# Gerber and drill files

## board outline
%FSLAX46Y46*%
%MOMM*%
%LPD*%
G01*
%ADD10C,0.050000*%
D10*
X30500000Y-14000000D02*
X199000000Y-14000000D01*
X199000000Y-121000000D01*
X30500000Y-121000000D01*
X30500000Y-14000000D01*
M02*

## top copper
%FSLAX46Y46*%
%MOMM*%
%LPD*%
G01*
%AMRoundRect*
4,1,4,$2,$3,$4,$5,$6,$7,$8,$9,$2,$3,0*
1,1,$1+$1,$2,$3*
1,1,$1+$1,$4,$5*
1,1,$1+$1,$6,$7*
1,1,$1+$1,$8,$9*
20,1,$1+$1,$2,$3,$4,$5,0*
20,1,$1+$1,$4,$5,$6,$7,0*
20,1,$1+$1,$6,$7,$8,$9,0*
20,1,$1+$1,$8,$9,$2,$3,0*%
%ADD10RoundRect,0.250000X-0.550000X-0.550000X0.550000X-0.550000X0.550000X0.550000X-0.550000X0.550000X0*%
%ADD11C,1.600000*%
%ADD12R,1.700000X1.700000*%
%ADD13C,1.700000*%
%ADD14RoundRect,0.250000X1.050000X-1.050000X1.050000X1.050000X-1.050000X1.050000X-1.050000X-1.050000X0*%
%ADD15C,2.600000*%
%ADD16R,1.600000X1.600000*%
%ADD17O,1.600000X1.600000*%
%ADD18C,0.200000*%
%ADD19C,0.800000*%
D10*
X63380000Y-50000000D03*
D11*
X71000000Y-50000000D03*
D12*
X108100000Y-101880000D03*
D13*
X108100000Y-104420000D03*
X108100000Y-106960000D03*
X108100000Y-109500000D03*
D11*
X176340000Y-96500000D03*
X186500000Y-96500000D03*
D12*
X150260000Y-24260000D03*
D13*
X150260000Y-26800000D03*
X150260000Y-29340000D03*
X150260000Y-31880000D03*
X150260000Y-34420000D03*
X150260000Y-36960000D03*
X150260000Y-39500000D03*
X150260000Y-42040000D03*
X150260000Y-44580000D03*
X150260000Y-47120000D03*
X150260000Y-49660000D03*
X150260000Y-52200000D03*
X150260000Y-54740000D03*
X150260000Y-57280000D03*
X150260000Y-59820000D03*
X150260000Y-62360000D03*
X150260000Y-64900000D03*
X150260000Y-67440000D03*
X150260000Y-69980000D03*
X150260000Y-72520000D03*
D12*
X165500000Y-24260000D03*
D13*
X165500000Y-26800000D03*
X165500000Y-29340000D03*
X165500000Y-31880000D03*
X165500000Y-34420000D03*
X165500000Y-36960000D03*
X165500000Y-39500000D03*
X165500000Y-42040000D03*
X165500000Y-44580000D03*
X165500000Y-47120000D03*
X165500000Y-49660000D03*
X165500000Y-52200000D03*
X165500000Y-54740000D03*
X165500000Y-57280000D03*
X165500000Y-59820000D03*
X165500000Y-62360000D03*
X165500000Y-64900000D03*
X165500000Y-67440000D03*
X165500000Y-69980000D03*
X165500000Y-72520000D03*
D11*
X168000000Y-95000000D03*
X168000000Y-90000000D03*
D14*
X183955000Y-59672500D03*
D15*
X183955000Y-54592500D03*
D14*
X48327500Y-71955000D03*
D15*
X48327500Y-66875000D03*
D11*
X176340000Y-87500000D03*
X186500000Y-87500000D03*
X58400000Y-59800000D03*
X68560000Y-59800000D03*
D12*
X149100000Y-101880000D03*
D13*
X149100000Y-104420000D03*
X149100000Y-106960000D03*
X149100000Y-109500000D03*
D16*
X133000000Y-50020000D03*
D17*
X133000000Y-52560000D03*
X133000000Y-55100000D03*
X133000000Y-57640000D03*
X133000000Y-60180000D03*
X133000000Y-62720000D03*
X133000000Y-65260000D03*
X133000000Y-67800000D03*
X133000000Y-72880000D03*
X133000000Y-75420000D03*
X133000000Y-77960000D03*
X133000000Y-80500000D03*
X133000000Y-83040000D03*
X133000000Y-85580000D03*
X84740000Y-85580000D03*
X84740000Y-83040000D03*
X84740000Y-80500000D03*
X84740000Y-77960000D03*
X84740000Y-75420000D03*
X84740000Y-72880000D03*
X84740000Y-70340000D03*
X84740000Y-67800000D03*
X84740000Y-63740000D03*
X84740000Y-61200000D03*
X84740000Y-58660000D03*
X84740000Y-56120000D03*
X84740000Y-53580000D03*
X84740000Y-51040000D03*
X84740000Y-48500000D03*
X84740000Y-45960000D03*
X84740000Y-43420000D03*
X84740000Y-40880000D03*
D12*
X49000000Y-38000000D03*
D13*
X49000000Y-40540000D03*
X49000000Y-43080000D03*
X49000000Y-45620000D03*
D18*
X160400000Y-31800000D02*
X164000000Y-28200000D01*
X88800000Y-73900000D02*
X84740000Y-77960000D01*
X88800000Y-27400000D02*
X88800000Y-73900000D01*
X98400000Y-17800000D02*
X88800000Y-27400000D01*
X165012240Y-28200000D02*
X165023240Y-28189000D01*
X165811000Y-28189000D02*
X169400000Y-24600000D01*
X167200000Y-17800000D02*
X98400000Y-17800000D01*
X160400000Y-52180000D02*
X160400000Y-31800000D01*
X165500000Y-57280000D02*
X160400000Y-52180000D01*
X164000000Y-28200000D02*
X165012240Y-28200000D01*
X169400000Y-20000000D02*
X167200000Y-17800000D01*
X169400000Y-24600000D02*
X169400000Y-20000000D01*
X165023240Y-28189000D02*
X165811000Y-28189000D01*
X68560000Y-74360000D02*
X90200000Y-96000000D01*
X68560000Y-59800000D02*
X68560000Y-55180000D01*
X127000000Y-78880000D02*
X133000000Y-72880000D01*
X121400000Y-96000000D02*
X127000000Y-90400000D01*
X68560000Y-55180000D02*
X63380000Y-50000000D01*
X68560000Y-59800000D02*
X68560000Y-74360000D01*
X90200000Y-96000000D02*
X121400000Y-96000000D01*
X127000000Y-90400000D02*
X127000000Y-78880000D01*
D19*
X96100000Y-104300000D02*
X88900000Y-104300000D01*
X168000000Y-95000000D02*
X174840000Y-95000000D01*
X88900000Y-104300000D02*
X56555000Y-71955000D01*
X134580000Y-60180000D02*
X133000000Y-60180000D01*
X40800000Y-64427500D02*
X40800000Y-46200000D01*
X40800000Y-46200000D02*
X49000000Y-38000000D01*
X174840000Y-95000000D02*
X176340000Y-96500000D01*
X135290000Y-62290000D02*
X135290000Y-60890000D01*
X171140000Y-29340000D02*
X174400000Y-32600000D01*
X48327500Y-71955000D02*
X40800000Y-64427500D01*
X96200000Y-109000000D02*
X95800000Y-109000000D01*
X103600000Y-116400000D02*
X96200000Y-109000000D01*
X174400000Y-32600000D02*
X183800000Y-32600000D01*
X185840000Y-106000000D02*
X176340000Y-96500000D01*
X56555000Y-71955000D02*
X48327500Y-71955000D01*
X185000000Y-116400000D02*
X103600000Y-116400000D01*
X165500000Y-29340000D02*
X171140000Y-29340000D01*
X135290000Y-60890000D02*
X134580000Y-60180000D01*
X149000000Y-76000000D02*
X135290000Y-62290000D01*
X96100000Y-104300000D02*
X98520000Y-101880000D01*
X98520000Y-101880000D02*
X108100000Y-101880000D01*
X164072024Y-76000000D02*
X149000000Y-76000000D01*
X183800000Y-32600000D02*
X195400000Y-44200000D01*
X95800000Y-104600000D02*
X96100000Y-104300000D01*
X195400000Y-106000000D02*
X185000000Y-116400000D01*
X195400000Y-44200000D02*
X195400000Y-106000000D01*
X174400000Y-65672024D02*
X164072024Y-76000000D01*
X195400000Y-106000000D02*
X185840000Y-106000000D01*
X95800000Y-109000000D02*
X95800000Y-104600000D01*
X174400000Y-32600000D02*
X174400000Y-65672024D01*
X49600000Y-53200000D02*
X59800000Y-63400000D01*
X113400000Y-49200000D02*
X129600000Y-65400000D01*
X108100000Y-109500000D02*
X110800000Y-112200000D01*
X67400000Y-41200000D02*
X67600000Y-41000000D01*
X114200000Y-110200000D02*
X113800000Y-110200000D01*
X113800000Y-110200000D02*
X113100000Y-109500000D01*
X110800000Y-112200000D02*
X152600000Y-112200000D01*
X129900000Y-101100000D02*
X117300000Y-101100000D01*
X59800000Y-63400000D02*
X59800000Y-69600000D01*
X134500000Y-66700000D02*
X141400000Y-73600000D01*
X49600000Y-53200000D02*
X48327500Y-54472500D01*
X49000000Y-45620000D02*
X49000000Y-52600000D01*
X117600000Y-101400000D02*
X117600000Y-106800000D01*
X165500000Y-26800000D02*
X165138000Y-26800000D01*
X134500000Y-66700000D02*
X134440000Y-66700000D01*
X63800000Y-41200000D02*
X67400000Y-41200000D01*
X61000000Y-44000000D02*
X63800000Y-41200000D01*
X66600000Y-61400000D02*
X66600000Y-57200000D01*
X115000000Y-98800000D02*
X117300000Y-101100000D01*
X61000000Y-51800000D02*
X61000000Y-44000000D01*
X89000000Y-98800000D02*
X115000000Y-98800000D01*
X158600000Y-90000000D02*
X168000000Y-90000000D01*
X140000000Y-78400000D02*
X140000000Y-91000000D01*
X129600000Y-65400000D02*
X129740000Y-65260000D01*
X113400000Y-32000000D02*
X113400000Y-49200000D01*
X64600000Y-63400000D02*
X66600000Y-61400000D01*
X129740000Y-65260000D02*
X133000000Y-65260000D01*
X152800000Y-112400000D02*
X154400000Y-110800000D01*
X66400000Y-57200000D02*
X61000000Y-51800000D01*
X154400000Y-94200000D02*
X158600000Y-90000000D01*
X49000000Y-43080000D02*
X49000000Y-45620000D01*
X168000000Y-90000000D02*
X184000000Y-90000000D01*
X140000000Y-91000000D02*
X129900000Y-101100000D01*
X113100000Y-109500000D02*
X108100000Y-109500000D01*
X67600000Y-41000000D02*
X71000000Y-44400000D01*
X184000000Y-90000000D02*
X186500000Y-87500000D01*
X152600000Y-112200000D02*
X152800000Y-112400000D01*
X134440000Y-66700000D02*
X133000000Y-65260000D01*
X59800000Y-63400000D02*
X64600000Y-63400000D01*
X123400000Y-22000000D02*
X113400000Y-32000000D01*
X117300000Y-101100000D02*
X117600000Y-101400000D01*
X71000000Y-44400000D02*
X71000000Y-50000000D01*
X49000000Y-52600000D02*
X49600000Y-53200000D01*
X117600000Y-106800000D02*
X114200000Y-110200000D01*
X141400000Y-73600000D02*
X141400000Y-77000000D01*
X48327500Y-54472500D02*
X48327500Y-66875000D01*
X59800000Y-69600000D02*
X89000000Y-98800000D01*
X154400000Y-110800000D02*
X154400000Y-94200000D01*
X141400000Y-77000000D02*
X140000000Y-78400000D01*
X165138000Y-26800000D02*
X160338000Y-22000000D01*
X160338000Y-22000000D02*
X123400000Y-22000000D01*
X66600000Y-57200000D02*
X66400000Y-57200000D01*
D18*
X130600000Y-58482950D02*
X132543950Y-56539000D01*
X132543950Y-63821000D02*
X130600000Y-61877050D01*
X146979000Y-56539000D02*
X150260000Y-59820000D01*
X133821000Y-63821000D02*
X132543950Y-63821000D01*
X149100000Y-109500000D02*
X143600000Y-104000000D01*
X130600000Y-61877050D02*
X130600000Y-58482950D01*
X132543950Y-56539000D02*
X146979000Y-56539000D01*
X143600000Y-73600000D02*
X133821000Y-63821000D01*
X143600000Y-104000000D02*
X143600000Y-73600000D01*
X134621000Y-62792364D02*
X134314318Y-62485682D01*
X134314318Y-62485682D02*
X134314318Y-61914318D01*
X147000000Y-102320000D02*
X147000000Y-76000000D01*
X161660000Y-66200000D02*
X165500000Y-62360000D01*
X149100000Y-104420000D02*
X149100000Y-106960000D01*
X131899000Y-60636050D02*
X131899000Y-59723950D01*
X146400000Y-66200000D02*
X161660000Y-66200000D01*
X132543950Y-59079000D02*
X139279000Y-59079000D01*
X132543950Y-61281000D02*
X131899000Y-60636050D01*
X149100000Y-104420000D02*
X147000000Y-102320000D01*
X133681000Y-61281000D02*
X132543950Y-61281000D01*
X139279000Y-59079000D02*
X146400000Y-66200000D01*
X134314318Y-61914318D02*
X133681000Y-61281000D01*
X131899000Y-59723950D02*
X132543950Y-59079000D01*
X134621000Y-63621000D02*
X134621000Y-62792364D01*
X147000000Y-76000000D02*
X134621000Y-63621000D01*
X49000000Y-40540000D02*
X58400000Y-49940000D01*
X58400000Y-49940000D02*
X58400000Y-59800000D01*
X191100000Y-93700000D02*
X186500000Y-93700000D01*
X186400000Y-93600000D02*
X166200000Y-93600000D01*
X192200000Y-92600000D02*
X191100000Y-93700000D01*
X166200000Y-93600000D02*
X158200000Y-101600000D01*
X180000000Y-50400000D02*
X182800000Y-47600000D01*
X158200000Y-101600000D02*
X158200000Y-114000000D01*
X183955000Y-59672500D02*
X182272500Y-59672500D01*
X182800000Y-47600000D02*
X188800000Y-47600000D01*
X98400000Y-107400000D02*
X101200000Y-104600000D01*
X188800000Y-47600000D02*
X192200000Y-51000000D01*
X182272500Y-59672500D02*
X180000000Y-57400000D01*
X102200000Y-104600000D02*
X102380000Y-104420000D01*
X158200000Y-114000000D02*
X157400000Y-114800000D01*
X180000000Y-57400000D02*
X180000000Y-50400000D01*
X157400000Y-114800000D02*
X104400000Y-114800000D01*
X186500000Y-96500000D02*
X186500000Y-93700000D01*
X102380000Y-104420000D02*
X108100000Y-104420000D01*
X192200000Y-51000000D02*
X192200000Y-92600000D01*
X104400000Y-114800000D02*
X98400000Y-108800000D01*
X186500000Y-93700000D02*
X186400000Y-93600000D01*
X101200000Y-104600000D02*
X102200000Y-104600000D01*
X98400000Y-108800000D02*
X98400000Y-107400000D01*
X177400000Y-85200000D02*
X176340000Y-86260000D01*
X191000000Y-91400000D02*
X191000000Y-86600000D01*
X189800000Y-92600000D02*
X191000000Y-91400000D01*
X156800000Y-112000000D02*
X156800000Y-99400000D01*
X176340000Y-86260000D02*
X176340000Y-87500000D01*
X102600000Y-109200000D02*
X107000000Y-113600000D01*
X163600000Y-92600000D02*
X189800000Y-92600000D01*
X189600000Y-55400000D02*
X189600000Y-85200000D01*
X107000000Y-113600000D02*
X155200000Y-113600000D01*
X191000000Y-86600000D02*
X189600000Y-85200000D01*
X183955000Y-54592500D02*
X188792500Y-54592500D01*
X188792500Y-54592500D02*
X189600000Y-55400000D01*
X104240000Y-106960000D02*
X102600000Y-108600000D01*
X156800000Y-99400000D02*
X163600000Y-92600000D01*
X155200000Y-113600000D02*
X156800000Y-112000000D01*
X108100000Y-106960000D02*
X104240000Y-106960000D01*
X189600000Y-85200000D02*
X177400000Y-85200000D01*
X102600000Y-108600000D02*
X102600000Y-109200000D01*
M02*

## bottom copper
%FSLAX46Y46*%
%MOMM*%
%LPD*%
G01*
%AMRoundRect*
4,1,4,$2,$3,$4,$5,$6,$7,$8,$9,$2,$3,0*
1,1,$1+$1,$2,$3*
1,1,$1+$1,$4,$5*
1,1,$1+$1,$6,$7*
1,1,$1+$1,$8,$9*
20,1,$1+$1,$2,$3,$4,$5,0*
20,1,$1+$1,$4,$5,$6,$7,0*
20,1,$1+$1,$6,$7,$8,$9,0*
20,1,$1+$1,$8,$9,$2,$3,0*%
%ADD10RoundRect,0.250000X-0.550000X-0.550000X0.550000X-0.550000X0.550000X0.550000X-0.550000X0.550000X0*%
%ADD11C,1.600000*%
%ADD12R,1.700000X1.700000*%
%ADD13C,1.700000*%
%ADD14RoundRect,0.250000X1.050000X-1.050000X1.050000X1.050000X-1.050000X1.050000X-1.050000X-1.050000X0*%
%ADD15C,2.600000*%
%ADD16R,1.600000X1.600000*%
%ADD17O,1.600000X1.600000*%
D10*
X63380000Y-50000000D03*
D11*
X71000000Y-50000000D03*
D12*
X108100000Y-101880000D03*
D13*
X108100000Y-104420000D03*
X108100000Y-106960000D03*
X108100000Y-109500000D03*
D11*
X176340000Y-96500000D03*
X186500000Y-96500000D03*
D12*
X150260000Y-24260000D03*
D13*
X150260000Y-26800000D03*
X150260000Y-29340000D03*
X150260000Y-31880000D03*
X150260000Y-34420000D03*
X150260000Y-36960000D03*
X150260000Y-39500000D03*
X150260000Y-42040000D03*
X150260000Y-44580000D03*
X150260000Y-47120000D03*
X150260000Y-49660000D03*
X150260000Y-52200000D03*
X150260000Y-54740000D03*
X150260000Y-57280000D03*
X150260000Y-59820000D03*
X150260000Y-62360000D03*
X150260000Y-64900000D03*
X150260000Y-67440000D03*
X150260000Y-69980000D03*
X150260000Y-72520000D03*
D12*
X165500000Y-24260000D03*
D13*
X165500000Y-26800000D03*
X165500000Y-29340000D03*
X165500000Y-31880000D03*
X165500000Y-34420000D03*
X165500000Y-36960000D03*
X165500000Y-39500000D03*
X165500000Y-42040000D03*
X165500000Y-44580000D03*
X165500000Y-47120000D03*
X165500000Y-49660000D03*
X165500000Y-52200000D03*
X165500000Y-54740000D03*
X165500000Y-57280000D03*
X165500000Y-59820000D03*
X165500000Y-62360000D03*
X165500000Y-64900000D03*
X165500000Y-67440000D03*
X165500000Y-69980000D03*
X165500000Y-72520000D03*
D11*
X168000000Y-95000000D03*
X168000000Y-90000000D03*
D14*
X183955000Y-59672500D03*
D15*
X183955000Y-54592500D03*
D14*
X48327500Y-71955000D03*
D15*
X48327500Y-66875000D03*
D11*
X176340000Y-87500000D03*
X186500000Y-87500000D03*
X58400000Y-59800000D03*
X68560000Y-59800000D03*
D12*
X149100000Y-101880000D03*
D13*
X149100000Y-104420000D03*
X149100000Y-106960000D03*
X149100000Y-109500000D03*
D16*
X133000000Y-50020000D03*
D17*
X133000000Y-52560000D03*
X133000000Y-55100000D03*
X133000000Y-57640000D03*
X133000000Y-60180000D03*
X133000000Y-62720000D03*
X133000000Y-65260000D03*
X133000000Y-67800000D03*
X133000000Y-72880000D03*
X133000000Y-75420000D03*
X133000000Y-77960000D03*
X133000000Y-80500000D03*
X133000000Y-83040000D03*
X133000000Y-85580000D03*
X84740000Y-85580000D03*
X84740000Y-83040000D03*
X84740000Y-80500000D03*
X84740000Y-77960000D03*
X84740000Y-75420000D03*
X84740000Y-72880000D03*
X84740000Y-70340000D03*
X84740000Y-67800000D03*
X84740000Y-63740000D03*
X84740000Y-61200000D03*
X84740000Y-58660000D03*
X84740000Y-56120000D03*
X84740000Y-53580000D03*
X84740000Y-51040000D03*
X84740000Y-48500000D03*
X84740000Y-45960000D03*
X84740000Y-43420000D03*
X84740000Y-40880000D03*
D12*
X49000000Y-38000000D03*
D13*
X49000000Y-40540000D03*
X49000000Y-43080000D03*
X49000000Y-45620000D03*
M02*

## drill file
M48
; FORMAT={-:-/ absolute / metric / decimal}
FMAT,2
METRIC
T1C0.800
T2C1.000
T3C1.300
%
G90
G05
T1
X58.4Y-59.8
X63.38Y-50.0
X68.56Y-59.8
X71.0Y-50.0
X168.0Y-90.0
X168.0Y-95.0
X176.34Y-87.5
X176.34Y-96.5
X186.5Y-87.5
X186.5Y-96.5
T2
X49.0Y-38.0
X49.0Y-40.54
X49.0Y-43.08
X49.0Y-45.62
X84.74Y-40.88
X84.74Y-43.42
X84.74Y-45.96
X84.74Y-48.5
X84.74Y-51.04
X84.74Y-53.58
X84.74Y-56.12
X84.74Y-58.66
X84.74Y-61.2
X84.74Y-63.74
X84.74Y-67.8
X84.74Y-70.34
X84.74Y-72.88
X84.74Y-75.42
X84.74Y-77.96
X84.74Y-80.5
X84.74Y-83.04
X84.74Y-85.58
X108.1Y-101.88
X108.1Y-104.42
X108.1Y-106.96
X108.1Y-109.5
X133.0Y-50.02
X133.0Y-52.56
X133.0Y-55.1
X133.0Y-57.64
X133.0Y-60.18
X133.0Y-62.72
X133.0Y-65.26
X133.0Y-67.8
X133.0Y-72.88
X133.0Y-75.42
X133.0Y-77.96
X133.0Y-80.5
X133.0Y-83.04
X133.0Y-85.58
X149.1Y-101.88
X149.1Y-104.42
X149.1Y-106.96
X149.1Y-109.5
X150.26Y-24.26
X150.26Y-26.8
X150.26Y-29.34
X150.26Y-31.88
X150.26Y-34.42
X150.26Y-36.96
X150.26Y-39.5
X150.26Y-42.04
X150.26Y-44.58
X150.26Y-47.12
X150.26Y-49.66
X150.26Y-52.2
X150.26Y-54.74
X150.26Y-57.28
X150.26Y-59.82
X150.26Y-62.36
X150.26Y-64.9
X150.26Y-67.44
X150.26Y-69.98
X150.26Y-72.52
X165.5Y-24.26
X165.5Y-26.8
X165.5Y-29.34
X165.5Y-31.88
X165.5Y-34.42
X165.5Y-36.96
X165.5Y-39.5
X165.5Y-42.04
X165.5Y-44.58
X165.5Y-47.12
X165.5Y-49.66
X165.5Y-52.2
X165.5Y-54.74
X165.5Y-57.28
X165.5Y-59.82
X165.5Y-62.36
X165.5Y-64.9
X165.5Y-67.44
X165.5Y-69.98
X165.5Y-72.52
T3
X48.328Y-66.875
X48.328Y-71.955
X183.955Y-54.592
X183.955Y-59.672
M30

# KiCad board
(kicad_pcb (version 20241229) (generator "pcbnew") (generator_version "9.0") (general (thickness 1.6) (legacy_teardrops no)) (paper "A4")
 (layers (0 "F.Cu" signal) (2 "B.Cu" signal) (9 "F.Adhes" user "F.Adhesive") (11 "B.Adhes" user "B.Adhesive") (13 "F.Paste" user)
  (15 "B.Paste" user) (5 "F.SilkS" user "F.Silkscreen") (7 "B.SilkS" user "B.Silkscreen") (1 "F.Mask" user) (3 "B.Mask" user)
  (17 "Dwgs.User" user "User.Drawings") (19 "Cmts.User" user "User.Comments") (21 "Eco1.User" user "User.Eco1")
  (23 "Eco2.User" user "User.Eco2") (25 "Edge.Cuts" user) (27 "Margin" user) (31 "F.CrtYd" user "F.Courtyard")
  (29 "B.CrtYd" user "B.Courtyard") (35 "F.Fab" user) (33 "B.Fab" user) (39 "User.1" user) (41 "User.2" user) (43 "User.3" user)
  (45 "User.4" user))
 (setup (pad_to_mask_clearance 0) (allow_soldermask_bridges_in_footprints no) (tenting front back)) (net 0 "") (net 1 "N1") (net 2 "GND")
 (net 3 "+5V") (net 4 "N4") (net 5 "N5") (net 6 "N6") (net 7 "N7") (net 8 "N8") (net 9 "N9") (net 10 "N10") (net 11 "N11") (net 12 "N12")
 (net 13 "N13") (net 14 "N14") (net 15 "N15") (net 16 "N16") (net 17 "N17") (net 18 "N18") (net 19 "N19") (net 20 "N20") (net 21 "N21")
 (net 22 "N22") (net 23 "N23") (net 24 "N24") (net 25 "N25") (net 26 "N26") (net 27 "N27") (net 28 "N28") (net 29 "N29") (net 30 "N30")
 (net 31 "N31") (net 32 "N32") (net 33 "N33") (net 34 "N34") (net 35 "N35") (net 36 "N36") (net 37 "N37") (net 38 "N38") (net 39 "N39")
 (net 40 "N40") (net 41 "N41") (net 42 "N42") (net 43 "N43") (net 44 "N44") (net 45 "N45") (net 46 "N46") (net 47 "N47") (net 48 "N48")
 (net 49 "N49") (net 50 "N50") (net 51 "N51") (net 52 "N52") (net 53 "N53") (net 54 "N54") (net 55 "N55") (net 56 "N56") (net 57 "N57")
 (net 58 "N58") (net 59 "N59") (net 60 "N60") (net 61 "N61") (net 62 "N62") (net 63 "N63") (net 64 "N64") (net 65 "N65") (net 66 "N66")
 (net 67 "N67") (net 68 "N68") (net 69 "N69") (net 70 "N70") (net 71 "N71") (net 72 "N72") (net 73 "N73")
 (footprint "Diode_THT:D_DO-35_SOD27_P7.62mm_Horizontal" (layer "F.Cu") (at 63.38 50)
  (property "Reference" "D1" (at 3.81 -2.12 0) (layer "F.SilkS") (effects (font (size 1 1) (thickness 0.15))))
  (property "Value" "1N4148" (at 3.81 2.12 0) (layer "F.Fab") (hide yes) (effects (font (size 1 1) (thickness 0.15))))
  (pad "1" thru_hole roundrect (at 0 0) (size 1.6 1.6) (drill 0.8) (layers "*.Cu" "*.Mask") (remove_unused_layers no)
   (roundrect_rratio 0.15625) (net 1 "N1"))
  (pad "2" thru_hole circle (at 7.62 0) (size 1.6 1.6) (drill 0.8) (layers "*.Cu" "*.Mask") (remove_unused_layers no) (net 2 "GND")))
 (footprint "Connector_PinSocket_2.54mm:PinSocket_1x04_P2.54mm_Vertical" (layer "F.Cu") (at 108.1 101.88)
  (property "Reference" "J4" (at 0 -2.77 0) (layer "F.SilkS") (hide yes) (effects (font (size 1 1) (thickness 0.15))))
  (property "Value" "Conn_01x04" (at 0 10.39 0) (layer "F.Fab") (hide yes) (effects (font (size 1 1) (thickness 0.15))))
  (pad "1" thru_hole rect (at 0 0) (size 1.7 1.7) (drill 1) (layers "*.Cu" "*.Mask") (remove_unused_layers no) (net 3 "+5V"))
  (pad "2" thru_hole circle (at 0 2.54) (size 1.7 1.7) (drill 1) (layers "*.Cu" "*.Mask") (remove_unused_layers no) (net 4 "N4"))
  (pad "3" thru_hole circle (at 0 5.08) (size 1.7 1.7) (drill 1) (layers "*.Cu" "*.Mask") (remove_unused_layers no) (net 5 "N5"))
  (pad "4" thru_hole circle (at 0 7.62) (size 1.7 1.7) (drill 1) (layers "*.Cu" "*.Mask") (remove_unused_layers no) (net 2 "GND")))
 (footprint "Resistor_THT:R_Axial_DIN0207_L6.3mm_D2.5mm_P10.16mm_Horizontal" (layer "F.Cu") (at 176.34 96.5)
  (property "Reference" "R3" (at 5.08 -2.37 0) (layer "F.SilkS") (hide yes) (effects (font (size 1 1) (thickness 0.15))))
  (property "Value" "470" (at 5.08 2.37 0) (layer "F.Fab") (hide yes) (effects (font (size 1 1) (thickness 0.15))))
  (pad "1" thru_hole circle (at 0 0) (size 1.6 1.6) (drill 0.8) (layers "*.Cu" "*.Mask") (remove_unused_layers no) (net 3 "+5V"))
  (pad "2" thru_hole circle (at 10.16 0) (size 1.6 1.6) (drill 0.8) (layers "*.Cu" "*.Mask") (remove_unused_layers no) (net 4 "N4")))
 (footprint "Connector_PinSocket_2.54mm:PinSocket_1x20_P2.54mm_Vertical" (layer "F.Cu") (at 150.26 24.26)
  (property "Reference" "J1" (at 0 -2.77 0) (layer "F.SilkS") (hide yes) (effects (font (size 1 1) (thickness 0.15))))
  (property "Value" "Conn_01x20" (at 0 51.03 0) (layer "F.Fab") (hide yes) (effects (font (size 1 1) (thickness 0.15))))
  (pad "1" thru_hole rect (at 0 0) (size 1.7 1.7) (drill 1) (layers "*.Cu" "*.Mask") (remove_unused_layers no) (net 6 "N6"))
  (pad "2" thru_hole circle (at 0 2.54) (size 1.7 1.7) (drill 1) (layers "*.Cu" "*.Mask") (remove_unused_layers no) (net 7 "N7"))
  (pad "3" thru_hole circle (at 0 5.08) (size 1.7 1.7) (drill 1) (layers "*.Cu" "*.Mask") (remove_unused_layers no) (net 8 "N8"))
  (pad "4" thru_hole circle (at 0 7.62) (size 1.7 1.7) (drill 1) (layers "*.Cu" "*.Mask") (remove_unused_layers no) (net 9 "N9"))
  (pad "5" thru_hole circle (at 0 10.16) (size 1.7 1.7) (drill 1) (layers "*.Cu" "*.Mask") (remove_unused_layers no) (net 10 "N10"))
  (pad "6" thru_hole circle (at 0 12.7) (size 1.7 1.7) (drill 1) (layers "*.Cu" "*.Mask") (remove_unused_layers no) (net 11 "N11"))
  (pad "7" thru_hole circle (at 0 15.24) (size 1.7 1.7) (drill 1) (layers "*.Cu" "*.Mask") (remove_unused_layers no) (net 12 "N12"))
  (pad "8" thru_hole circle (at 0 17.78) (size 1.7 1.7) (drill 1) (layers "*.Cu" "*.Mask") (remove_unused_layers no) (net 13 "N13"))
  (pad "9" thru_hole circle (at 0 20.32) (size 1.7 1.7) (drill 1) (layers "*.Cu" "*.Mask") (remove_unused_layers no) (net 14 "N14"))
  (pad "10" thru_hole circle (at 0 22.86) (size 1.7 1.7) (drill 1) (layers "*.Cu" "*.Mask") (remove_unused_layers no) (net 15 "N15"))
  (pad "11" thru_hole circle (at 0 25.4) (size 1.7 1.7) (drill 1) (layers "*.Cu" "*.Mask") (remove_unused_layers no) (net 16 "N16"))
  (pad "12" thru_hole circle (at 0 27.94) (size 1.7 1.7) (drill 1) (layers "*.Cu" "*.Mask") (remove_unused_layers no) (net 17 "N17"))
  (pad "13" thru_hole circle (at 0 30.48) (size 1.7 1.7) (drill 1) (layers "*.Cu" "*.Mask") (remove_unused_layers no) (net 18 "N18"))
  (pad "14" thru_hole circle (at 0 33.02) (size 1.7 1.7) (drill 1) (layers "*.Cu" "*.Mask") (remove_unused_layers no) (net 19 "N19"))
  (pad "15" thru_hole circle (at 0 35.56) (size 1.7 1.7) (drill 1) (layers "*.Cu" "*.Mask") (remove_unused_layers no) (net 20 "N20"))
  (pad "16" thru_hole circle (at 0 38.1) (size 1.7 1.7) (drill 1) (layers "*.Cu" "*.Mask") (remove_unused_layers no) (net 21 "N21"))
  (pad "17" thru_hole circle (at 0 40.64) (size 1.7 1.7) (drill 1) (layers "*.Cu" "*.Mask") (remove_unused_layers no) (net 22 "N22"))
  (pad "18" thru_hole circle (at 0 43.18) (size 1.7 1.7) (drill 1) (layers "*.Cu" "*.Mask") (remove_unused_layers no) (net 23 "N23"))
  (pad "19" thru_hole circle (at 0 45.72) (size 1.7 1.7) (drill 1) (layers "*.Cu" "*.Mask") (remove_unused_layers no) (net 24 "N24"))
  (pad "20" thru_hole circle (at 0 48.26) (size 1.7 1.7) (drill 1) (layers "*.Cu" "*.Mask") (remove_unused_layers no) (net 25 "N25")))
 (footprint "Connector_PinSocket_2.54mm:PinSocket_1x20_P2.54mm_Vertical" (layer "F.Cu") (at 165.5 24.26)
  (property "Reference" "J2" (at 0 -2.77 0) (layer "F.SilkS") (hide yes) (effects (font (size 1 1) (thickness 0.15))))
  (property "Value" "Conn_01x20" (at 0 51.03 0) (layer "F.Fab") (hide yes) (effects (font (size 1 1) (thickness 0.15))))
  (pad "1" thru_hole rect (at 0 0) (size 1.7 1.7) (drill 1) (layers "*.Cu" "*.Mask") (remove_unused_layers no) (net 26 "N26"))
  (pad "2" thru_hole circle (at 0 2.54) (size 1.7 1.7) (drill 1) (layers "*.Cu" "*.Mask") (remove_unused_layers no) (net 2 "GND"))
  (pad "3" thru_hole circle (at 0 5.08) (size 1.7 1.7) (drill 1) (layers "*.Cu" "*.Mask") (remove_unused_layers no) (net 3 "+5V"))
  (pad "4" thru_hole circle (at 0 7.62) (size 1.7 1.7) (drill 1) (layers "*.Cu" "*.Mask") (remove_unused_layers no) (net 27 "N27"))
  (pad "5" thru_hole circle (at 0 10.16) (size 1.7 1.7) (drill 1) (layers "*.Cu" "*.Mask") (remove_unused_layers no) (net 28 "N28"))
  (pad "6" thru_hole circle (at 0 12.7) (size 1.7 1.7) (drill 1) (layers "*.Cu" "*.Mask") (remove_unused_layers no) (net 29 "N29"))
  (pad "7" thru_hole circle (at 0 15.24) (size 1.7 1.7) (drill 1) (layers "*.Cu" "*.Mask") (remove_unused_layers no) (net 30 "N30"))
  (pad "8" thru_hole circle (at 0 17.78) (size 1.7 1.7) (drill 1) (layers "*.Cu" "*.Mask") (remove_unused_layers no) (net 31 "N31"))
  (pad "9" thru_hole circle (at 0 20.32) (size 1.7 1.7) (drill 1) (layers "*.Cu" "*.Mask") (remove_unused_layers no) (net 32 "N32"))
  (pad "10" thru_hole circle (at 0 22.86) (size 1.7 1.7) (drill 1) (layers "*.Cu" "*.Mask") (remove_unused_layers no) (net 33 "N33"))
  (pad "11" thru_hole circle (at 0 25.4) (size 1.7 1.7) (drill 1) (layers "*.Cu" "*.Mask") (remove_unused_layers no) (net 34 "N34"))
  (pad "12" thru_hole circle (at 0 27.94) (size 1.7 1.7) (drill 1) (layers "*.Cu" "*.Mask") (remove_unused_layers no) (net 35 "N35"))
  (pad "13" thru_hole circle (at 0 30.48) (size 1.7 1.7) (drill 1) (layers "*.Cu" "*.Mask") (remove_unused_layers no) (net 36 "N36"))
  (pad "14" thru_hole circle (at 0 33.02) (size 1.7 1.7) (drill 1) (layers "*.Cu" "*.Mask") (remove_unused_layers no) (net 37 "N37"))
  (pad "15" thru_hole circle (at 0 35.56) (size 1.7 1.7) (drill 1) (layers "*.Cu" "*.Mask") (remove_unused_layers no) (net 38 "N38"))
  (pad "16" thru_hole circle (at 0 38.1) (size 1.7 1.7) (drill 1) (layers "*.Cu" "*.Mask") (remove_unused_layers no) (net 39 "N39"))
  (pad "17" thru_hole circle (at 0 40.64) (size 1.7 1.7) (drill 1) (layers "*.Cu" "*.Mask") (remove_unused_layers no) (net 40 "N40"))
  (pad "18" thru_hole circle (at 0 43.18) (size 1.7 1.7) (drill 1) (layers "*.Cu" "*.Mask") (remove_unused_layers no) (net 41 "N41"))
  (pad "19" thru_hole circle (at 0 45.72) (size 1.7 1.7) (drill 1) (layers "*.Cu" "*.Mask") (remove_unused_layers no) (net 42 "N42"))
  (pad "20" thru_hole circle (at 0 48.26) (size 1.7 1.7) (drill 1) (layers "*.Cu" "*.Mask") (remove_unused_layers no) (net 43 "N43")))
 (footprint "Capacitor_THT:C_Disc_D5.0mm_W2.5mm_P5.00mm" (layer "F.Cu") (at 168 95 90)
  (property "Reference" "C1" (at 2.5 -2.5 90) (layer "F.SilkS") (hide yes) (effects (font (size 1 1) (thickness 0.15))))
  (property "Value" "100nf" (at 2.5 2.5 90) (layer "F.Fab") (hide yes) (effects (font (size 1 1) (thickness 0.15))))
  (pad "1" thru_hole circle (at 0 0 90) (size 1.6 1.6) (drill 0.8) (layers "*.Cu" "*.Mask") (remove_unused_layers no) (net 3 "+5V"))
  (pad "2" thru_hole circle (at 5 0 90) (size 1.6 1.6) (drill 0.8) (layers "*.Cu" "*.Mask") (remove_unused_layers no) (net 2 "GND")))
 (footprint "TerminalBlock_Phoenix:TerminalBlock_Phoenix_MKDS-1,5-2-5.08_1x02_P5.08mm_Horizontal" (layer "F.Cu") (at 183.955 59.6725 90)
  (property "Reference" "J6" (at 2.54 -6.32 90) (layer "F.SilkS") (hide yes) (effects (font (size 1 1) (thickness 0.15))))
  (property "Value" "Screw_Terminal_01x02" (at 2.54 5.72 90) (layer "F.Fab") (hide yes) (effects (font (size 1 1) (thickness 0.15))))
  (pad "1" thru_hole roundrect (at 0 0 90) (size 2.6 2.6) (drill 1.3) (layers "*.Cu" "*.Mask") (remove_unused_layers no)
   (roundrect_rratio 0.096154) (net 4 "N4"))
  (pad "2" thru_hole circle (at 5.08 0 90) (size 2.6 2.6) (drill 1.3) (layers "*.Cu" "*.Mask") (remove_unused_layers no) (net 5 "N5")))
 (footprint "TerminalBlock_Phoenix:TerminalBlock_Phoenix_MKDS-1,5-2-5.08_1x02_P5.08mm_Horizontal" (layer "F.Cu") (at 48.3275 71.955 90)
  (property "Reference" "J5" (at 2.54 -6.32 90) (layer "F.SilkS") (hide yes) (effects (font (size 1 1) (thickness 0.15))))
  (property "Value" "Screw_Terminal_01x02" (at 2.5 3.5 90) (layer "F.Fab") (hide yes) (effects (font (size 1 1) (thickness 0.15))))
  (pad "1" thru_hole roundrect (at 0 0 90) (size 2.6 2.6) (drill 1.3) (layers "*.Cu" "*.Mask") (remove_unused_layers no)
   (roundrect_rratio 0.096154) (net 3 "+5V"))
  (pad "2" thru_hole circle (at 5.08 0 90) (size 2.6 2.6) (drill 1.3) (layers "*.Cu" "*.Mask") (remove_unused_layers no) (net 2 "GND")))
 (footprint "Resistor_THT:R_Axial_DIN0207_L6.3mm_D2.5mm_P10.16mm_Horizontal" (layer "F.Cu") (at 176.34 87.5)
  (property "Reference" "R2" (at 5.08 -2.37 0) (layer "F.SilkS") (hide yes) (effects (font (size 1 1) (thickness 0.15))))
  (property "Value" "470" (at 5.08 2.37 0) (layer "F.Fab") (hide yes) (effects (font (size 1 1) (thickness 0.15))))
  (pad "1" thru_hole circle (at 0 0) (size 1.6 1.6) (drill 0.8) (layers "*.Cu" "*.Mask") (remove_unused_layers no) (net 5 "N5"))
  (pad "2" thru_hole circle (at 10.16 0) (size 1.6 1.6) (drill 0.8) (layers "*.Cu" "*.Mask") (remove_unused_layers no) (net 2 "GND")))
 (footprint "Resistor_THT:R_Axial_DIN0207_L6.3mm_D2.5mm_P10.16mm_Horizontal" (layer "F.Cu") (at 58.4 59.8)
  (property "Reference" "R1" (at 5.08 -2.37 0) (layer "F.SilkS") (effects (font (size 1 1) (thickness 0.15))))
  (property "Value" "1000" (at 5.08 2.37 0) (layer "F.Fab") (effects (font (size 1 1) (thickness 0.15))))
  (pad "1" thru_hole circle (at 0 0) (size 1.6 1.6) (drill 0.8) (layers "*.Cu" "*.Mask") (remove_unused_layers no) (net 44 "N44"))
  (pad "2" thru_hole circle (at 10.16 0) (size 1.6 1.6) (drill 0.8) (layers "*.Cu" "*.Mask") (remove_unused_layers no) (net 1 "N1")))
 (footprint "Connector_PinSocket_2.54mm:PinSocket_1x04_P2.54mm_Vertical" (layer "F.Cu") (at 149.1 101.88)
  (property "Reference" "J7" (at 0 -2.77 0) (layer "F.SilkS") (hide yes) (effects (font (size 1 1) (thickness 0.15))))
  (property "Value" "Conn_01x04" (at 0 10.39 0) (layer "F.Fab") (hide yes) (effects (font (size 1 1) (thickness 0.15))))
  (pad "1" thru_hole rect (at 0 0) (size 1.7 1.7) (drill 1) (layers "*.Cu" "*.Mask") (remove_unused_layers no) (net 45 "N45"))
  (pad "2" thru_hole circle (at 0 2.54) (size 1.7 1.7) (drill 1) (layers "*.Cu" "*.Mask") (remove_unused_layers no) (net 39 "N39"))
  (pad "3" thru_hole circle (at 0 5.08) (size 1.7 1.7) (drill 1) (layers "*.Cu" "*.Mask") (remove_unused_layers no) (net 39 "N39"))
  (pad "4" thru_hole circle (at 0 7.62) (size 1.7 1.7) (drill 1) (layers "*.Cu" "*.Mask") (remove_unused_layers no) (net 20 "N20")))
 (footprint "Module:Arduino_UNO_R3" (layer "F.Cu") (at 133 50.02 -90)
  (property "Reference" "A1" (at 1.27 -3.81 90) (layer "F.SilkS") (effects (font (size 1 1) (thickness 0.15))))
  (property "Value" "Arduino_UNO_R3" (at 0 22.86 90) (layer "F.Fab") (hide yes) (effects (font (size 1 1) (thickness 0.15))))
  (pad "1" thru_hole rect (at 0 0) (size 1.6 1.6) (drill 1) (layers "*.Cu" "*.Mask") (remove_unused_layers no) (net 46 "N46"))
  (pad "2" thru_hole oval (at 2.54 0) (size 1.6 1.6) (drill 1) (layers "*.Cu" "*.Mask") (remove_unused_layers no) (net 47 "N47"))
  (pad "3" thru_hole oval (at 5.08 0) (size 1.6 1.6) (drill 1) (layers "*.Cu" "*.Mask") (remove_unused_layers no) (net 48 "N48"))
  (pad "4" thru_hole oval (at 7.62 0) (size 1.6 1.6) (drill 1) (layers "*.Cu" "*.Mask") (remove_unused_layers no) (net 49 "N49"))
  (pad "5" thru_hole oval (at 10.16 0) (size 1.6 1.6) (drill 1) (layers "*.Cu" "*.Mask") (remove_unused_layers no) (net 3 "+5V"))
  (pad "6" thru_hole oval (at 12.7 0) (size 1.6 1.6) (drill 1) (layers "*.Cu" "*.Mask") (remove_unused_layers no) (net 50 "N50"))
  (pad "7" thru_hole oval (at 15.24 0) (size 1.6 1.6) (drill 1) (layers "*.Cu" "*.Mask") (remove_unused_layers no) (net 2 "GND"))
  (pad "8" thru_hole oval (at 17.78 0) (size 1.6 1.6) (drill 1) (layers "*.Cu" "*.Mask") (remove_unused_layers no) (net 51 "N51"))
  (pad "9" thru_hole oval (at 22.86 0) (size 1.6 1.6) (drill 1) (layers "*.Cu" "*.Mask") (remove_unused_layers no) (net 1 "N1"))
  (pad "10" thru_hole oval (at 25.4 0) (size 1.6 1.6) (drill 1) (layers "*.Cu" "*.Mask") (remove_unused_layers no) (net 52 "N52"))
  (pad "11" thru_hole oval (at 27.94 0) (size 1.6 1.6) (drill 1) (layers "*.Cu" "*.Mask") (remove_unused_layers no) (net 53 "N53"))
  (pad "12" thru_hole oval (at 30.48 0) (size 1.6 1.6) (drill 1) (layers "*.Cu" "*.Mask") (remove_unused_layers no) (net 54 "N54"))
  (pad "13" thru_hole oval (at 33.02 0) (size 1.6 1.6) (drill 1) (layers "*.Cu" "*.Mask") (remove_unused_layers no) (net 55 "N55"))
  (pad "14" thru_hole oval (at 35.56 0) (size 1.6 1.6) (drill 1) (layers "*.Cu" "*.Mask") (remove_unused_layers no) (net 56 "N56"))
  (pad "15" thru_hole oval (at 35.56 48.26) (size 1.6 1.6) (drill 1) (layers "*.Cu" "*.Mask") (remove_unused_layers no) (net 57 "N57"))
  (pad "16" thru_hole oval (at 33.02 48.26) (size 1.6 1.6) (drill 1) (layers "*.Cu" "*.Mask") (remove_unused_layers no) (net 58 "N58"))
  (pad "17" thru_hole oval (at 30.48 48.26) (size 1.6 1.6) (drill 1) (layers "*.Cu" "*.Mask") (remove_unused_layers no) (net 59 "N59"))
  (pad "18" thru_hole oval (at 27.94 48.26) (size 1.6 1.6) (drill 1) (layers "*.Cu" "*.Mask") (remove_unused_layers no) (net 37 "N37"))
  (pad "19" thru_hole oval (at 25.4 48.26) (size 1.6 1.6) (drill 1) (layers "*.Cu" "*.Mask") (remove_unused_layers no) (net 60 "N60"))
  (pad "20" thru_hole oval (at 22.86 48.26) (size 1.6 1.6) (drill 1) (layers "*.Cu" "*.Mask") (remove_unused_layers no) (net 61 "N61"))
  (pad "21" thru_hole oval (at 20.32 48.26) (size 1.6 1.6) (drill 1) (layers "*.Cu" "*.Mask") (remove_unused_layers no) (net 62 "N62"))
  (pad "22" thru_hole oval (at 17.78 48.26) (size 1.6 1.6) (drill 1) (layers "*.Cu" "*.Mask") (remove_unused_layers no) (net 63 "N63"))
  (pad "23" thru_hole oval (at 13.72 48.26) (size 1.6 1.6) (drill 1) (layers "*.Cu" "*.Mask") (remove_unused_layers no) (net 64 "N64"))
  (pad "24" thru_hole oval (at 11.18 48.26) (size 1.6 1.6) (drill 1) (layers "*.Cu" "*.Mask") (remove_unused_layers no) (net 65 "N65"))
  (pad "25" thru_hole oval (at 8.64 48.26) (size 1.6 1.6) (drill 1) (layers "*.Cu" "*.Mask") (remove_unused_layers no) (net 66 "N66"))
  (pad "26" thru_hole oval (at 6.1 48.26) (size 1.6 1.6) (drill 1) (layers "*.Cu" "*.Mask") (remove_unused_layers no) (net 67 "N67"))
  (pad "27" thru_hole oval (at 3.56 48.26) (size 1.6 1.6) (drill 1) (layers "*.Cu" "*.Mask") (remove_unused_layers no) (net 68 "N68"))
  (pad "28" thru_hole oval (at 1.02 48.26) (size 1.6 1.6) (drill 1) (layers "*.Cu" "*.Mask") (remove_unused_layers no) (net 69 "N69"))
  (pad "29" thru_hole oval (at -1.52 48.26) (size 1.6 1.6) (drill 1) (layers "*.Cu" "*.Mask") (remove_unused_layers no) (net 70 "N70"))
  (pad "30" thru_hole oval (at -4.06 48.26) (size 1.6 1.6) (drill 1) (layers "*.Cu" "*.Mask") (remove_unused_layers no) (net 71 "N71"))
  (pad "31" thru_hole oval (at -6.6 48.26) (size 1.6 1.6) (drill 1) (layers "*.Cu" "*.Mask") (remove_unused_layers no) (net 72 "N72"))
  (pad "32" thru_hole oval (at -9.14 48.26) (size 1.6 1.6) (drill 1) (layers "*.Cu" "*.Mask") (remove_unused_layers no) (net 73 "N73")))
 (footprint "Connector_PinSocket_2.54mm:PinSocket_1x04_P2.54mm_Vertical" (layer "F.Cu") (at 49 38)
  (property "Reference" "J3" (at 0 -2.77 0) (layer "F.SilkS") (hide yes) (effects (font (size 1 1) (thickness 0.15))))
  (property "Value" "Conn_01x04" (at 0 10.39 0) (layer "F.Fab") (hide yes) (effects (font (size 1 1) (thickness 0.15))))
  (pad "1" thru_hole rect (at 0 0) (size 1.7 1.7) (drill 1) (layers "*.Cu" "*.Mask") (remove_unused_layers no) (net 3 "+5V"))
  (pad "2" thru_hole circle (at 0 2.54) (size 1.7 1.7) (drill 1) (layers "*.Cu" "*.Mask") (remove_unused_layers no) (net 44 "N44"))
  (pad "3" thru_hole circle (at 0 5.08) (size 1.7 1.7) (drill 1) (layers "*.Cu" "*.Mask") (remove_unused_layers no) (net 2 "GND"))
  (pad "4" thru_hole circle (at 0 7.62) (size 1.7 1.7) (drill 1) (layers "*.Cu" "*.Mask") (remove_unused_layers no) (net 2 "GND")))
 (gr_rect (start 30.5 14) (end 199 121) (stroke (width 0.05) (type default)) (fill no) (layer "Edge.Cuts"))
 (segment (start 160.4 31.8) (end 164 28.2) (width 0.2) (layer "F.Cu") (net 37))
 (segment (start 88.8 73.9) (end 84.74 77.96) (width 0.2) (layer "F.Cu") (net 37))
 (segment (start 88.8 27.4) (end 88.8 73.9) (width 0.2) (layer "F.Cu") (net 37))
 (segment (start 98.4 17.8) (end 88.8 27.4) (width 0.2) (layer "F.Cu") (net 37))
 (segment (start 165.01224 28.2) (end 165.02324 28.189) (width 0.2) (layer "F.Cu") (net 37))
 (segment (start 165.811 28.189) (end 169.4 24.6) (width 0.2) (layer "F.Cu") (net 37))
 (segment (start 167.2 17.8) (end 98.4 17.8) (width 0.2) (layer "F.Cu") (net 37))
 (segment (start 160.4 52.18) (end 160.4 31.8) (width 0.2) (layer "F.Cu") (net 37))
 (segment (start 165.5 57.28) (end 160.4 52.18) (width 0.2) (layer "F.Cu") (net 37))
 (segment (start 164 28.2) (end 165.01224 28.2) (width 0.2) (layer "F.Cu") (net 37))
 (segment (start 169.4 20) (end 167.2 17.8) (width 0.2) (layer "F.Cu") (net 37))
 (segment (start 169.4 24.6) (end 169.4 20) (width 0.2) (layer "F.Cu") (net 37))
 (segment (start 165.02324 28.189) (end 165.811 28.189) (width 0.2) (layer "F.Cu") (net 37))
 (segment (start 68.56 74.36) (end 90.2 96) (width 0.2) (layer "F.Cu") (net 1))
 (segment (start 68.56 59.8) (end 68.56 55.18) (width 0.2) (layer "F.Cu") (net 1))
 (segment (start 127 78.88) (end 133 72.88) (width 0.2) (layer "F.Cu") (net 1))
 (segment (start 121.4 96) (end 127 90.4) (width 0.2) (layer "F.Cu") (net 1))
 (segment (start 68.56 55.18) (end 63.38 50) (width 0.2) (layer "F.Cu") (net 1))
 (segment (start 68.56 59.8) (end 68.56 74.36) (width 0.2) (layer "F.Cu") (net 1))
 (segment (start 90.2 96) (end 121.4 96) (width 0.2) (layer "F.Cu") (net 1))
 (segment (start 127 90.4) (end 127 78.88) (width 0.2) (layer "F.Cu") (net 1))
 (segment (start 96.1 104.3) (end 88.9 104.3) (width 0.8) (layer "F.Cu") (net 3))
 (segment (start 168 95) (end 174.84 95) (width 0.8) (layer "F.Cu") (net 3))
 (segment (start 88.9 104.3) (end 56.555 71.955) (width 0.8) (layer "F.Cu") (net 3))
 (segment (start 134.58 60.18) (end 133 60.18) (width 0.8) (layer "F.Cu") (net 3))
 (segment (start 40.8 64.4275) (end 40.8 46.2) (width 0.8) (layer "F.Cu") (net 3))
 (segment (start 40.8 46.2) (end 49 38) (width 0.8) (layer "F.Cu") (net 3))
 (segment (start 174.84 95) (end 176.34 96.5) (width 0.8) (layer "F.Cu") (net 3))
 (segment (start 135.29 62.29) (end 135.29 60.89) (width 0.8) (layer "F.Cu") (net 3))
 (segment (start 171.14 29.34) (end 174.4 32.6) (width 0.8) (layer "F.Cu") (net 3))
 (segment (start 48.3275 71.955) (end 40.8 64.4275) (width 0.8) (layer "F.Cu") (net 3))
 (segment (start 96.2 109) (end 95.8 109) (width 0.8) (layer "F.Cu") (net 3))
 (segment (start 103.6 116.4) (end 96.2 109) (width 0.8) (layer "F.Cu") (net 3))
 (segment (start 174.4 32.6) (end 183.8 32.6) (width 0.8) (layer "F.Cu") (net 3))
 (segment (start 185.84 106) (end 176.34 96.5) (width 0.8) (layer "F.Cu") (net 3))
 (segment (start 56.555 71.955) (end 48.3275 71.955) (width 0.8) (layer "F.Cu") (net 3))
 (segment (start 185 116.4) (end 103.6 116.4) (width 0.8) (layer "F.Cu") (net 3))
 (segment (start 165.5 29.34) (end 171.14 29.34) (width 0.8) (layer "F.Cu") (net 3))
 (segment (start 135.29 60.89) (end 134.58 60.18) (width 0.8) (layer "F.Cu") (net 3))
 (segment (start 149 76) (end 135.29 62.29) (width 0.8) (layer "F.Cu") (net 3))
 (segment (start 96.1 104.3) (end 98.52 101.88) (width 0.8) (layer "F.Cu") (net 3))
 (segment (start 98.52 101.88) (end 108.1 101.88) (width 0.8) (layer "F.Cu") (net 3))
 (segment (start 164.072024 76) (end 149 76) (width 0.8) (layer "F.Cu") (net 3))
 (segment (start 183.8 32.6) (end 195.4 44.2) (width 0.8) (layer "F.Cu") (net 3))
 (segment (start 95.8 104.6) (end 96.1 104.3) (width 0.8) (layer "F.Cu") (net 3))
 (segment (start 195.4 106) (end 185 116.4) (width 0.8) (layer "F.Cu") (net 3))
 (segment (start 195.4 44.2) (end 195.4 106) (width 0.8) (layer "F.Cu") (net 3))
 (segment (start 174.4 65.672024) (end 164.072024 76) (width 0.8) (layer "F.Cu") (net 3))
 (segment (start 195.4 106) (end 185.84 106) (width 0.8) (layer "F.Cu") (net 3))
 (segment (start 95.8 109) (end 95.8 104.6) (width 0.8) (layer "F.Cu") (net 3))
 (segment (start 174.4 32.6) (end 174.4 65.672024) (width 0.8) (layer "F.Cu") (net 3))
 (segment (start 49.6 53.2) (end 59.8 63.4) (width 0.8) (layer "F.Cu") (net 2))
 (segment (start 113.4 49.2) (end 129.6 65.4) (width 0.8) (layer "F.Cu") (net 2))
 (segment (start 108.1 109.5) (end 110.8 112.2) (width 0.8) (layer "F.Cu") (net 2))
 (segment (start 67.4 41.2) (end 67.6 41) (width 0.8) (layer "F.Cu") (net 2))
 (segment (start 114.2 110.2) (end 113.8 110.2) (width 0.8) (layer "F.Cu") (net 2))
 (segment (start 113.8 110.2) (end 113.1 109.5) (width 0.8) (layer "F.Cu") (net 2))
 (segment (start 110.8 112.2) (end 152.6 112.2) (width 0.8) (layer "F.Cu") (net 2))
 (segment (start 129.9 101.1) (end 117.3 101.1) (width 0.8) (layer "F.Cu") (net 2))
 (segment (start 59.8 63.4) (end 59.8 69.6) (width 0.8) (layer "F.Cu") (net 2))
 (segment (start 134.5 66.7) (end 141.4 73.6) (width 0.8) (layer "F.Cu") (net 2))
 (segment (start 49.6 53.2) (end 48.3275 54.4725) (width 0.8) (layer "F.Cu") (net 2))
 (segment (start 49 45.62) (end 49 52.6) (width 0.8) (layer "F.Cu") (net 2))
 (segment (start 117.6 101.4) (end 117.6 106.8) (width 0.8) (layer "F.Cu") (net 2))
 (segment (start 165.5 26.8) (end 165.138 26.8) (width 0.8) (layer "F.Cu") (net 2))
 (segment (start 134.5 66.7) (end 134.44 66.7) (width 0.8) (layer "F.Cu") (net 2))
 (segment (start 63.8 41.2) (end 67.4 41.2) (width 0.8) (layer "F.Cu") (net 2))
 (segment (start 61 44) (end 63.8 41.2) (width 0.8) (layer "F.Cu") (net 2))
 (segment (start 66.6 61.4) (end 66.6 57.2) (width 0.8) (layer "F.Cu") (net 2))
 (segment (start 115 98.8) (end 117.3 101.1) (width 0.8) (layer "F.Cu") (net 2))
 (segment (start 61 51.8) (end 61 44) (width 0.8) (layer "F.Cu") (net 2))
 (segment (start 89 98.8) (end 115 98.8) (width 0.8) (layer "F.Cu") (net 2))
 (segment (start 158.6 90) (end 168 90) (width 0.8) (layer "F.Cu") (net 2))
 (segment (start 140 78.4) (end 140 91) (width 0.8) (layer "F.Cu") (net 2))
 (segment (start 129.6 65.4) (end 129.74 65.26) (width 0.8) (layer "F.Cu") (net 2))
 (segment (start 113.4 32) (end 113.4 49.2) (width 0.8) (layer "F.Cu") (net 2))
 (segment (start 64.6 63.4) (end 66.6 61.4) (width 0.8) (layer "F.Cu") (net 2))
 (segment (start 129.74 65.26) (end 133 65.26) (width 0.8) (layer "F.Cu") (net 2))
 (segment (start 152.8 112.4) (end 154.4 110.8) (width 0.8) (layer "F.Cu") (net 2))
 (segment (start 66.4 57.2) (end 61 51.8) (width 0.8) (layer "F.Cu") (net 2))
 (segment (start 154.4 94.2) (end 158.6 90) (width 0.8) (layer "F.Cu") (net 2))
 (segment (start 49 43.08) (end 49 45.62) (width 0.8) (layer "F.Cu") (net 2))
 (segment (start 168 90) (end 184 90) (width 0.8) (layer "F.Cu") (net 2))
 (segment (start 140 91) (end 129.9 101.1) (width 0.8) (layer "F.Cu") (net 2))
 (segment (start 113.1 109.5) (end 108.1 109.5) (width 0.8) (layer "F.Cu") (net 2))
 (segment (start 67.6 41) (end 71 44.4) (width 0.8) (layer "F.Cu") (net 2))
 (segment (start 184 90) (end 186.5 87.5) (width 0.8) (layer "F.Cu") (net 2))
 (segment (start 152.6 112.2) (end 152.8 112.4) (width 0.8) (layer "F.Cu") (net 2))
 (segment (start 134.44 66.7) (end 133 65.26) (width 0.8) (layer "F.Cu") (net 2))
 (segment (start 59.8 63.4) (end 64.6 63.4) (width 0.8) (layer "F.Cu") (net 2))
 (segment (start 123.4 22) (end 113.4 32) (width 0.8) (layer "F.Cu") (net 2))
 (segment (start 117.3 101.1) (end 117.6 101.4) (width 0.8) (layer "F.Cu") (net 2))
 (segment (start 71 44.4) (end 71 50) (width 0.8) (layer "F.Cu") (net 2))
 (segment (start 49 52.6) (end 49.6 53.2) (width 0.8) (layer "F.Cu") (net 2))
 (segment (start 117.6 106.8) (end 114.2 110.2) (width 0.8) (layer "F.Cu") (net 2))
 (segment (start 141.4 73.6) (end 141.4 77) (width 0.8) (layer "F.Cu") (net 2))
 (segment (start 48.3275 54.4725) (end 48.3275 66.875) (width 0.8) (layer "F.Cu") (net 2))
 (segment (start 59.8 69.6) (end 89 98.8) (width 0.8) (layer "F.Cu") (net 2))
 (segment (start 154.4 110.8) (end 154.4 94.2) (width 0.8) (layer "F.Cu") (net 2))
 (segment (start 141.4 77) (end 140 78.4) (width 0.8) (layer "F.Cu") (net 2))
 (segment (start 165.138 26.8) (end 160.338 22) (width 0.8) (layer "F.Cu") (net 2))
 (segment (start 160.338 22) (end 123.4 22) (width 0.8) (layer "F.Cu") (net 2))
 (segment (start 66.6 57.2) (end 66.4 57.2) (width 0.8) (layer "F.Cu") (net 2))
 (segment (start 130.6 58.48295) (end 132.54395 56.539) (width 0.2) (layer "F.Cu") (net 20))
 (segment (start 132.54395 63.821) (end 130.6 61.87705) (width 0.2) (layer "F.Cu") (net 20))
 (segment (start 146.979 56.539) (end 150.26 59.82) (width 0.2) (layer "F.Cu") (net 20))
 (segment (start 133.821 63.821) (end 132.54395 63.821) (width 0.2) (layer "F.Cu") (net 20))
 (segment (start 149.1 109.5) (end 143.6 104) (width 0.2) (layer "F.Cu") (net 20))
 (segment (start 130.6 61.87705) (end 130.6 58.48295) (width 0.2) (layer "F.Cu") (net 20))
 (segment (start 132.54395 56.539) (end 146.979 56.539) (width 0.2) (layer "F.Cu") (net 20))
 (segment (start 143.6 73.6) (end 133.821 63.821) (width 0.2) (layer "F.Cu") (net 20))
 (segment (start 143.6 104) (end 143.6 73.6) (width 0.2) (layer "F.Cu") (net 20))
 (segment (start 134.621 62.792364) (end 134.314318 62.485682) (width 0.2) (layer "F.Cu") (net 39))
 (segment (start 134.314318 62.485682) (end 134.314318 61.914318) (width 0.2) (layer "F.Cu") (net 39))
 (segment (start 147 102.32) (end 147 76) (width 0.2) (layer "F.Cu") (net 39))
 (segment (start 161.66 66.2) (end 165.5 62.36) (width 0.2) (layer "F.Cu") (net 39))
 (segment (start 149.1 104.42) (end 149.1 106.96) (width 0.2) (layer "F.Cu") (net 39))
 (segment (start 131.899 60.63605) (end 131.899 59.72395) (width 0.2) (layer "F.Cu") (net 39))
 (segment (start 146.4 66.2) (end 161.66 66.2) (width 0.2) (layer "F.Cu") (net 39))
 (segment (start 132.54395 59.079) (end 139.279 59.079) (width 0.2) (layer "F.Cu") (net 39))
 (segment (start 132.54395 61.281) (end 131.899 60.63605) (width 0.2) (layer "F.Cu") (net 39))
 (segment (start 149.1 104.42) (end 147 102.32) (width 0.2) (layer "F.Cu") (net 39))
 (segment (start 133.681 61.281) (end 132.54395 61.281) (width 0.2) (layer "F.Cu") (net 39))
 (segment (start 139.279 59.079) (end 146.4 66.2) (width 0.2) (layer "F.Cu") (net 39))
 (segment (start 134.314318 61.914318) (end 133.681 61.281) (width 0.2) (layer "F.Cu") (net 39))
 (segment (start 131.899 59.72395) (end 132.54395 59.079) (width 0.2) (layer "F.Cu") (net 39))
 (segment (start 134.621 63.621) (end 134.621 62.792364) (width 0.2) (layer "F.Cu") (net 39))
 (segment (start 147 76) (end 134.621 63.621) (width 0.2) (layer "F.Cu") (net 39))
 (segment (start 49 40.54) (end 58.4 49.94) (width 0.2) (layer "F.Cu") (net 44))
 (segment (start 58.4 49.94) (end 58.4 59.8) (width 0.2) (layer "F.Cu") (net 44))
 (segment (start 191.1 93.7) (end 186.5 93.7) (width 0.2) (layer "F.Cu") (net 4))
 (segment (start 186.4 93.6) (end 166.2 93.6) (width 0.2) (layer "F.Cu") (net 4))
 (segment (start 192.2 92.6) (end 191.1 93.7) (width 0.2) (layer "F.Cu") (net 4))
 (segment (start 166.2 93.6) (end 158.2 101.6) (width 0.2) (layer "F.Cu") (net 4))
 (segment (start 180 50.4) (end 182.8 47.6) (width 0.2) (layer "F.Cu") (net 4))
 (segment (start 158.2 101.6) (end 158.2 114) (width 0.2) (layer "F.Cu") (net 4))
 (segment (start 183.955 59.6725) (end 182.2725 59.6725) (width 0.2) (layer "F.Cu") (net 4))
 (segment (start 182.8 47.6) (end 188.8 47.6) (width 0.2) (layer "F.Cu") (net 4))
 (segment (start 98.4 107.4) (end 101.2 104.6) (width 0.2) (layer "F.Cu") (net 4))
 (segment (start 188.8 47.6) (end 192.2 51) (width 0.2) (layer "F.Cu") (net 4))
 (segment (start 182.2725 59.6725) (end 180 57.4) (width 0.2) (layer "F.Cu") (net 4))
 (segment (start 102.2 104.6) (end 102.38 104.42) (width 0.2) (layer "F.Cu") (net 4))
 (segment (start 158.2 114) (end 157.4 114.8) (width 0.2) (layer "F.Cu") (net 4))
 (segment (start 180 57.4) (end 180 50.4) (width 0.2) (layer "F.Cu") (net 4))
 (segment (start 157.4 114.8) (end 104.4 114.8) (width 0.2) (layer "F.Cu") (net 4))
 (segment (start 186.5 96.5) (end 186.5 93.7) (width 0.2) (layer "F.Cu") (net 4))
 (segment (start 102.38 104.42) (end 108.1 104.42) (width 0.2) (layer "F.Cu") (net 4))
 (segment (start 192.2 51) (end 192.2 92.6) (width 0.2) (layer "F.Cu") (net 4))
 (segment (start 104.4 114.8) (end 98.4 108.8) (width 0.2) (layer "F.Cu") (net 4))
 (segment (start 186.5 93.7) (end 186.4 93.6) (width 0.2) (layer "F.Cu") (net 4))
 (segment (start 101.2 104.6) (end 102.2 104.6) (width 0.2) (layer "F.Cu") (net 4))
 (segment (start 98.4 108.8) (end 98.4 107.4) (width 0.2) (layer "F.Cu") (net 4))
 (segment (start 177.4 85.2) (end 176.34 86.26) (width 0.2) (layer "F.Cu") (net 5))
 (segment (start 191 91.4) (end 191 86.6) (width 0.2) (layer "F.Cu") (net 5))
 (segment (start 189.8 92.6) (end 191 91.4) (width 0.2) (layer "F.Cu") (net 5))
 (segment (start 156.8 112) (end 156.8 99.4) (width 0.2) (layer "F.Cu") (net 5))
 (segment (start 176.34 86.26) (end 176.34 87.5) (width 0.2) (layer "F.Cu") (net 5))
 (segment (start 102.6 109.2) (end 107 113.6) (width 0.2) (layer "F.Cu") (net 5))
 (segment (start 163.6 92.6) (end 189.8 92.6) (width 0.2) (layer "F.Cu") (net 5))
 (segment (start 189.6 55.4) (end 189.6 85.2) (width 0.2) (layer "F.Cu") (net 5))
 (segment (start 107 113.6) (end 155.2 113.6) (width 0.2) (layer "F.Cu") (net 5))
 (segment (start 191 86.6) (end 189.6 85.2) (width 0.2) (layer "F.Cu") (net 5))
 (segment (start 183.955 54.5925) (end 188.7925 54.5925) (width 0.2) (layer "F.Cu") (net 5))
 (segment (start 188.7925 54.5925) (end 189.6 55.4) (width 0.2) (layer "F.Cu") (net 5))
 (segment (start 104.24 106.96) (end 102.6 108.6) (width 0.2) (layer "F.Cu") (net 5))
 (segment (start 156.8 99.4) (end 163.6 92.6) (width 0.2) (layer "F.Cu") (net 5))
 (segment (start 155.2 113.6) (end 156.8 112) (width 0.2) (layer "F.Cu") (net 5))
 (segment (start 108.1 106.96) (end 104.24 106.96) (width 0.2) (layer "F.Cu") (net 5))
 (segment (start 189.6 85.2) (end 177.4 85.2) (width 0.2) (layer "F.Cu") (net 5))
 (segment (start 102.6 108.6) (end 102.6 109.2) (width 0.2) (layer "F.Cu") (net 5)))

